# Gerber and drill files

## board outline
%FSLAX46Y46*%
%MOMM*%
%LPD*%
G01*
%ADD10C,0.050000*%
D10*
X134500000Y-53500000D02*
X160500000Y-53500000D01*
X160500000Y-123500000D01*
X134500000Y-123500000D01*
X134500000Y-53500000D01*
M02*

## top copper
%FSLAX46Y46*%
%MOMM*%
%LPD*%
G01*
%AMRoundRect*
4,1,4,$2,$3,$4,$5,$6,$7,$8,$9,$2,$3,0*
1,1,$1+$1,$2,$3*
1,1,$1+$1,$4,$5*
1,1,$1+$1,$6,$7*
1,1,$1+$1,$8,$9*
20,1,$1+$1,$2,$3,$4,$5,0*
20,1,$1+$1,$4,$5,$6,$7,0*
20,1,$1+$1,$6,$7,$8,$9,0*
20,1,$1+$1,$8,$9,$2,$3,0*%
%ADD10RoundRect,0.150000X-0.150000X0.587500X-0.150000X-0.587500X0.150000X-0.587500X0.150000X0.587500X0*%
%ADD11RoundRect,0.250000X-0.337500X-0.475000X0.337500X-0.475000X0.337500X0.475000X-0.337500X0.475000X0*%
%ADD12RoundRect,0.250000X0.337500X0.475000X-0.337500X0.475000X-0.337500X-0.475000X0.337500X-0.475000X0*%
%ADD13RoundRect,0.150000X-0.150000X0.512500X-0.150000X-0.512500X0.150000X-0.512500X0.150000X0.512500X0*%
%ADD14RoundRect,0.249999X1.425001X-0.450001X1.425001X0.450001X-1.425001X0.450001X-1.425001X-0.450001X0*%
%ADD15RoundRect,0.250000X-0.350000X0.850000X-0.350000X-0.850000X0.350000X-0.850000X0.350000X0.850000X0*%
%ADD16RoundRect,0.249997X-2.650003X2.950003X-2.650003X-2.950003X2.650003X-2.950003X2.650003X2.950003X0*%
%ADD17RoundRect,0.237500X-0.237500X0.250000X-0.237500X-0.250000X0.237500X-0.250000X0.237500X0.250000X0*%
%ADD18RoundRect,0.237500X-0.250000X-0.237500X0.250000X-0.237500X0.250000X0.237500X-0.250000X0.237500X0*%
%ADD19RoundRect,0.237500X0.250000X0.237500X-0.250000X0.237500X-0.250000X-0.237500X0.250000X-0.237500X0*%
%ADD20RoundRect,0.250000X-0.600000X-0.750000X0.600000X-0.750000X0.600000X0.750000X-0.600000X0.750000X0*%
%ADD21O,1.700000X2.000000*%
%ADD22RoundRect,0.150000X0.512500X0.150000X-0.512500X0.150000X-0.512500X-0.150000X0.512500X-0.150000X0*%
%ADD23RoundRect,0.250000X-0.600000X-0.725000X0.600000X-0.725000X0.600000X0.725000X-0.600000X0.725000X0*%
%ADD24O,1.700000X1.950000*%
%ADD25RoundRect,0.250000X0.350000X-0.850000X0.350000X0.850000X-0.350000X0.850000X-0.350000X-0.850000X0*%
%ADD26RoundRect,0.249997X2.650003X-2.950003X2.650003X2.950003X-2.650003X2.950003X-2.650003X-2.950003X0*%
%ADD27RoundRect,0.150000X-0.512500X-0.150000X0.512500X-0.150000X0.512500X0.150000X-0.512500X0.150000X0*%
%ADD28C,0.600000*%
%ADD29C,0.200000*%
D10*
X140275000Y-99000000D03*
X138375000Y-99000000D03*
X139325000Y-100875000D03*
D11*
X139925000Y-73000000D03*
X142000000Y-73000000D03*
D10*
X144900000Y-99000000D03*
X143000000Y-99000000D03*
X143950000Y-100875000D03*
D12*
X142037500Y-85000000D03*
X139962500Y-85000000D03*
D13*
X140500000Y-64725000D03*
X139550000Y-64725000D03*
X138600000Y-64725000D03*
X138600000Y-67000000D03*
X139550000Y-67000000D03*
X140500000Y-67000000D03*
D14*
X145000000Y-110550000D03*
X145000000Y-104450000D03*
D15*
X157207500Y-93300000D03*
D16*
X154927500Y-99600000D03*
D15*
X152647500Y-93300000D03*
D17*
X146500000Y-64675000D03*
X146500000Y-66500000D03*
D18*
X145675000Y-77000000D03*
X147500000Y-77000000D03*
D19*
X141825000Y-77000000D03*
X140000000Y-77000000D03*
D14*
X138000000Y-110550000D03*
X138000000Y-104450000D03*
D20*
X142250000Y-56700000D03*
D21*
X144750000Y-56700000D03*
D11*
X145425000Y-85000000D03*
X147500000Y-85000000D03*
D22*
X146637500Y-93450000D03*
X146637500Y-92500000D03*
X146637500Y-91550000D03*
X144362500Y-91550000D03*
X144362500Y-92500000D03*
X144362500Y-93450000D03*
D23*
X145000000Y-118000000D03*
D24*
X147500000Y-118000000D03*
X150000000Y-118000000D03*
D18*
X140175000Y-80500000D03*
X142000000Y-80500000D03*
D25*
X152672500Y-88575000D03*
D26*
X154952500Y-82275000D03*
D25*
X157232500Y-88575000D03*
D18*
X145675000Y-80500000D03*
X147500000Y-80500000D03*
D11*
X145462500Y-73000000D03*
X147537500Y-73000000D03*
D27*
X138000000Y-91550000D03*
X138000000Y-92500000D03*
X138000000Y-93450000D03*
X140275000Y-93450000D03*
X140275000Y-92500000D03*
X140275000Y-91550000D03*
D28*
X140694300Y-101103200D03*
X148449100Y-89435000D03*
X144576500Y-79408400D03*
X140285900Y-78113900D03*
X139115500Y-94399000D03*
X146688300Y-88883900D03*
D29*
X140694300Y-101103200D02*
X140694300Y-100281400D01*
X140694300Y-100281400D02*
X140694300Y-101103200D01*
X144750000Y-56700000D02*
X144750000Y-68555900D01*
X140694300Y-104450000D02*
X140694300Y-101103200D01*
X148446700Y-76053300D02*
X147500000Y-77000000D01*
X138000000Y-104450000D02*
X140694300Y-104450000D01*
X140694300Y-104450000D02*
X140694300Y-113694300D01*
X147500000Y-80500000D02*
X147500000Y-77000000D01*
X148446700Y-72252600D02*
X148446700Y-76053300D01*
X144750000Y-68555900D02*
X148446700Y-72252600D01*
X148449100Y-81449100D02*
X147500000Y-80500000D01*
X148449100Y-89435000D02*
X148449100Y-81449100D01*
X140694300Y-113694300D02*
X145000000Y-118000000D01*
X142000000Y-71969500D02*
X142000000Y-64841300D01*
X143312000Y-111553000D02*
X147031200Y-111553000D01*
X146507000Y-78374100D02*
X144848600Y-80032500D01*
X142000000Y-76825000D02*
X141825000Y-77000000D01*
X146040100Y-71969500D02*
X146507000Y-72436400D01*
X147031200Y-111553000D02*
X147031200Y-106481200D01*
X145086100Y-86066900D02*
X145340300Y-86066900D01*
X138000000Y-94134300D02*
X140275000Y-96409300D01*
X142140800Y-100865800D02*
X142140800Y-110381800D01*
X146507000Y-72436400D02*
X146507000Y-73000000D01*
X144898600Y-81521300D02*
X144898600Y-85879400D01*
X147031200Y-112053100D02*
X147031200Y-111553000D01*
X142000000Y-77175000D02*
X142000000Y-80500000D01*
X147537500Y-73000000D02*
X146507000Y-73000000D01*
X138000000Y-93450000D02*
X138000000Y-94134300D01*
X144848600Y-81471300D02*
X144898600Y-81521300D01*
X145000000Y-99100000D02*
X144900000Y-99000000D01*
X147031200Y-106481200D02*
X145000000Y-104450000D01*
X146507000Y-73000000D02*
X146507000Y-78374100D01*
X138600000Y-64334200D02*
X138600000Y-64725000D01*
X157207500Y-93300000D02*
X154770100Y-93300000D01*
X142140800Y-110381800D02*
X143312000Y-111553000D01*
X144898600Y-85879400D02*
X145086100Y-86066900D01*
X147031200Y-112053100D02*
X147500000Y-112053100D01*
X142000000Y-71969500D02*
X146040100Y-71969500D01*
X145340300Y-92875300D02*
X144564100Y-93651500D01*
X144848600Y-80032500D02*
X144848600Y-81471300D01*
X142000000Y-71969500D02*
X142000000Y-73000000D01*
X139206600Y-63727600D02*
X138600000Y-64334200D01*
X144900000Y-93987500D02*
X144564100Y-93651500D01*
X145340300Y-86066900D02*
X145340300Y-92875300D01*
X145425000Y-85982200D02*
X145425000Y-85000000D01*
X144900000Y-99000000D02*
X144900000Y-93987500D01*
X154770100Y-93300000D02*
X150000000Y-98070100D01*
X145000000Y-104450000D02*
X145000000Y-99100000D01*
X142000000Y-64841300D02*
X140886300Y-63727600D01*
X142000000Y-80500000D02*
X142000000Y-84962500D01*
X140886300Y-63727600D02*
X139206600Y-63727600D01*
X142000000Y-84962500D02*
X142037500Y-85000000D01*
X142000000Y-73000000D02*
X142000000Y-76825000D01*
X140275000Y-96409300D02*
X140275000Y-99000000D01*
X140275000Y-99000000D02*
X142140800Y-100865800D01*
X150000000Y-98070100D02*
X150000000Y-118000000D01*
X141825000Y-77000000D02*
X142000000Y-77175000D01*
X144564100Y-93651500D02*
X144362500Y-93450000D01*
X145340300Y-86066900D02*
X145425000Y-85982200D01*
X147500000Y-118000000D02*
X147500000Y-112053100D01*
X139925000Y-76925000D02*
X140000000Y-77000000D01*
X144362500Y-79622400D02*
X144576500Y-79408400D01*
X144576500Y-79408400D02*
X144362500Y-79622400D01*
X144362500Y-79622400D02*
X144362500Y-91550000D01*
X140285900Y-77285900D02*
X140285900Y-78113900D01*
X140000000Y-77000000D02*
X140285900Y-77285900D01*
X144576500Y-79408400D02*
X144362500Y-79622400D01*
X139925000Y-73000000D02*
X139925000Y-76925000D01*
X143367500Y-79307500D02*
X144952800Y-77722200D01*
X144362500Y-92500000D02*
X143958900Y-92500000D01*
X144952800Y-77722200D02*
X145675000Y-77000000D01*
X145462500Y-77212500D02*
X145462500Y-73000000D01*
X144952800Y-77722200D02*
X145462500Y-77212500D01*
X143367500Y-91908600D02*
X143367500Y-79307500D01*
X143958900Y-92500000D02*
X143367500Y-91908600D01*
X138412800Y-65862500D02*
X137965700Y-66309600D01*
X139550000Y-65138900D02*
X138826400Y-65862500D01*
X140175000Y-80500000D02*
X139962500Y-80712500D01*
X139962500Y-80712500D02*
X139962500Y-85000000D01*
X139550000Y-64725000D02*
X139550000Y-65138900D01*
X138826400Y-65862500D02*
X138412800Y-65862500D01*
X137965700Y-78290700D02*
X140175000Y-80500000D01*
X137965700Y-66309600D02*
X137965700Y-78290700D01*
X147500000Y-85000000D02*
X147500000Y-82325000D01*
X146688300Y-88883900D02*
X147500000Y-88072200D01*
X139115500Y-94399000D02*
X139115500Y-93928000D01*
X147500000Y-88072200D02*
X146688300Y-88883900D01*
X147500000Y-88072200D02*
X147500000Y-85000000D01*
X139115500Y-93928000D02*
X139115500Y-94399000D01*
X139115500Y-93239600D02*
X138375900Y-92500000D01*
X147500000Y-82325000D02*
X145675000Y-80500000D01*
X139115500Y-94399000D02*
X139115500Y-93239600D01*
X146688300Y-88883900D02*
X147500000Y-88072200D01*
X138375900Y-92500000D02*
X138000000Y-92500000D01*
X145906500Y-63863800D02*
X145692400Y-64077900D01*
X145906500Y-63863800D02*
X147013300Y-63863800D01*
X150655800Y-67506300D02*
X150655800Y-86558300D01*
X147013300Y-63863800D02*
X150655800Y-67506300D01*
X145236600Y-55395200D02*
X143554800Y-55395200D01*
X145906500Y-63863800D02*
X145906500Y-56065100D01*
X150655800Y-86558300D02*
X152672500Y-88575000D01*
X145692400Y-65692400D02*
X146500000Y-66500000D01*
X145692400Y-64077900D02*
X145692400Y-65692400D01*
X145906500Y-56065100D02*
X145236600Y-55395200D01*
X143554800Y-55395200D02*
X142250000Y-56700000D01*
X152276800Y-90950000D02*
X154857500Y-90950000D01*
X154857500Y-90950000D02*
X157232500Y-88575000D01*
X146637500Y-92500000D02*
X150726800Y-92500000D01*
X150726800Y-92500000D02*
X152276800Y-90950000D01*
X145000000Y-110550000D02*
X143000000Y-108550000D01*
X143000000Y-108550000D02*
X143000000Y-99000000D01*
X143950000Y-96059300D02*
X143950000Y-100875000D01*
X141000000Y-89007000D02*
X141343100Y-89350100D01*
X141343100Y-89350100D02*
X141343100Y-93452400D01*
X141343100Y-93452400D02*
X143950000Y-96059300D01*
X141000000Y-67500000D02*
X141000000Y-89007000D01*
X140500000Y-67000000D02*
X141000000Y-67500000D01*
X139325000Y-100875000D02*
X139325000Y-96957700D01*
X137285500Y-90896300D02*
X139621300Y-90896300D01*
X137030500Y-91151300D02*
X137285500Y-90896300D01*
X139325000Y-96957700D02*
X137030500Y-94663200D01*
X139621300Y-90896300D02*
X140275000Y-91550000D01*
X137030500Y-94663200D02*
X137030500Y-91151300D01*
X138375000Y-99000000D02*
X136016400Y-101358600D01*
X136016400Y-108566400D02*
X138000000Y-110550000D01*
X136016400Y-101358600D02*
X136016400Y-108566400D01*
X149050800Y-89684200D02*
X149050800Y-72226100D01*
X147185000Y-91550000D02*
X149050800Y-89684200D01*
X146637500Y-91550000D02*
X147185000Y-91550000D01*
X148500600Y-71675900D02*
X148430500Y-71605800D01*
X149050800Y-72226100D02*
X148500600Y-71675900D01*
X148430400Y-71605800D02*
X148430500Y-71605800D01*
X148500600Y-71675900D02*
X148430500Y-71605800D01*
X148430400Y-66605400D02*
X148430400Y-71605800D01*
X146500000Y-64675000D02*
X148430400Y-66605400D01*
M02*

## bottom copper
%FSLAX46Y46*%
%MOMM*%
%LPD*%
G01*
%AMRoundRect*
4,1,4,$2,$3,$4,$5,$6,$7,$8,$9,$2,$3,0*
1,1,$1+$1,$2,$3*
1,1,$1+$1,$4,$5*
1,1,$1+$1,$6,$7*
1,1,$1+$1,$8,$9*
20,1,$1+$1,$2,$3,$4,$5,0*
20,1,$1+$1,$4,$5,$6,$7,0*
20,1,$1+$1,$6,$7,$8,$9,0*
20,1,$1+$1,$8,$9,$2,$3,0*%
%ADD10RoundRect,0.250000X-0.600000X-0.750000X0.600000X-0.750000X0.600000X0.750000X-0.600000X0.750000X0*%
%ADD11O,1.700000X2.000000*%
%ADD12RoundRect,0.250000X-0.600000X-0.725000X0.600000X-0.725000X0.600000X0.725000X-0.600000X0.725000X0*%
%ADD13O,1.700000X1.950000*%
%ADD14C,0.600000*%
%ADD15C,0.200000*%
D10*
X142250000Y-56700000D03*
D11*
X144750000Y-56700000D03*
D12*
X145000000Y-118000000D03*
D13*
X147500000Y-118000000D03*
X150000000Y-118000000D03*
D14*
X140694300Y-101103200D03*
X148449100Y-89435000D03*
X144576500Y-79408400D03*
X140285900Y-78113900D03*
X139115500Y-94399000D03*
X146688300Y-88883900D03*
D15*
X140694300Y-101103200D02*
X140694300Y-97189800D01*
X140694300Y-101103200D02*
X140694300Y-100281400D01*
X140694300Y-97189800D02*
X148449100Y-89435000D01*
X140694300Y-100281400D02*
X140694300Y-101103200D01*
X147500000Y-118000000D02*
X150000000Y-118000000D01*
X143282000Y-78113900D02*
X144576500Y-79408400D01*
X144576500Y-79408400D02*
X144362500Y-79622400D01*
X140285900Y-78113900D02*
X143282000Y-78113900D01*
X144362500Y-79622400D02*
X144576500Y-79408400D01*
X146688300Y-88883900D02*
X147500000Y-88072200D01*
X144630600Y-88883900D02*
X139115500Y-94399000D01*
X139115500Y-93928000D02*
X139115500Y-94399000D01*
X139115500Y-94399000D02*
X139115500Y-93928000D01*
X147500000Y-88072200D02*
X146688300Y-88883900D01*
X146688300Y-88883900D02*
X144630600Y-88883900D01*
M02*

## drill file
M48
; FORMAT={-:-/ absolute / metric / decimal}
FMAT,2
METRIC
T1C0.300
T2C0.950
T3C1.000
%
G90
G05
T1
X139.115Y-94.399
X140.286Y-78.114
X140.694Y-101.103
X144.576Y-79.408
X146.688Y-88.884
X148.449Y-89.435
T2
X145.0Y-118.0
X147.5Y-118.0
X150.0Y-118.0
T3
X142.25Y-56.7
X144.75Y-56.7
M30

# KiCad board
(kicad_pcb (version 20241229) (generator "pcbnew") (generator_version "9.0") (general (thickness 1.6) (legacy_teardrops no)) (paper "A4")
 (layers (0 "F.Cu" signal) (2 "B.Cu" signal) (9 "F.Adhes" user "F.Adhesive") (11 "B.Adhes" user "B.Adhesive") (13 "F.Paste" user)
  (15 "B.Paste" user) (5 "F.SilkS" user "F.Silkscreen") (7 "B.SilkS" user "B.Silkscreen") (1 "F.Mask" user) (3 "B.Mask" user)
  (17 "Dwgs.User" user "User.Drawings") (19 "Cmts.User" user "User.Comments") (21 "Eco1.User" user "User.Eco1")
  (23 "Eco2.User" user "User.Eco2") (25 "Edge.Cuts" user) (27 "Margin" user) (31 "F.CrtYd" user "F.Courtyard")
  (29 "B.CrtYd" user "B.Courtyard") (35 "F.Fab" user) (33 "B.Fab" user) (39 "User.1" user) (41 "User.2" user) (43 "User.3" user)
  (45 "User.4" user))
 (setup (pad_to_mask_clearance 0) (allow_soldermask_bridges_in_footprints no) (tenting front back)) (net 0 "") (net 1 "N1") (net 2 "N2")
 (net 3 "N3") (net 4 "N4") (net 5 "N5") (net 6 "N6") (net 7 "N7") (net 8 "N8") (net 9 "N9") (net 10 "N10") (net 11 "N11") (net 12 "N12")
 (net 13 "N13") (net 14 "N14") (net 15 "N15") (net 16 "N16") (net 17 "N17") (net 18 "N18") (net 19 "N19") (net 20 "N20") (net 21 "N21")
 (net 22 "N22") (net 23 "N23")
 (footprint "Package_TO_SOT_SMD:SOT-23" (layer "F.Cu") (at 139.325 99.9375 -90)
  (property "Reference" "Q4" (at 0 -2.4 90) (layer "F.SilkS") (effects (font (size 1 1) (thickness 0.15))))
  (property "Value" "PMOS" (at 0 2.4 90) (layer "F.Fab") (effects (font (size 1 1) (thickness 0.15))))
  (pad "1" smd roundrect (at -0.9375 -0.95 270) (size 1.475 0.6) (layers "F.Cu" "F.Mask" "F.Paste") (roundrect_rratio 0.25) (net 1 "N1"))
  (pad "2" smd roundrect (at -0.9375 0.95 270) (size 1.475 0.6) (layers "F.Cu" "F.Mask" "F.Paste") (roundrect_rratio 0.25) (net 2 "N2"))
  (pad "3" smd roundrect (at 0.9375 0 270) (size 1.475 0.6) (layers "F.Cu" "F.Mask" "F.Paste") (roundrect_rratio 0.25) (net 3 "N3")))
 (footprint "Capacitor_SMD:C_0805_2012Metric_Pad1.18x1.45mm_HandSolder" (layer "F.Cu") (at 140.9625 73)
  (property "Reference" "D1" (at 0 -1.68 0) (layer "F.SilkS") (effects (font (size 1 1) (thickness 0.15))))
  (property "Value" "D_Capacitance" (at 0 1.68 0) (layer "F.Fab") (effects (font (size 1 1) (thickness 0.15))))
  (pad "1" smd roundrect (at -1.0375 0) (size 1.175 1.45) (layers "F.Cu" "F.Mask" "F.Paste") (roundrect_rratio 0.212766) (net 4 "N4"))
  (pad "2" smd roundrect (at 1.0375 0) (size 1.175 1.45) (layers "F.Cu" "F.Mask" "F.Paste") (roundrect_rratio 0.212766) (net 1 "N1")))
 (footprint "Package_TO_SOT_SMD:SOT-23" (layer "F.Cu") (at 143.95 99.9375 -90)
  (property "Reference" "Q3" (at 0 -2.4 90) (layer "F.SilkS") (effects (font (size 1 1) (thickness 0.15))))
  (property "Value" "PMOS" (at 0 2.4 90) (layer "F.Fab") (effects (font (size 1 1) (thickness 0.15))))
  (pad "1" smd roundrect (at -0.9375 -0.95 270) (size 1.475 0.6) (layers "F.Cu" "F.Mask" "F.Paste") (roundrect_rratio 0.25) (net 1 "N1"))
  (pad "2" smd roundrect (at -0.9375 0.95 270) (size 1.475 0.6) (layers "F.Cu" "F.Mask" "F.Paste") (roundrect_rratio 0.25) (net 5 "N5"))
  (pad "3" smd roundrect (at 0.9375 0 270) (size 1.475 0.6) (layers "F.Cu" "F.Mask" "F.Paste") (roundrect_rratio 0.25) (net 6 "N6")))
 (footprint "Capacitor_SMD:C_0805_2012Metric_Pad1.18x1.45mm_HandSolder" (layer "F.Cu") (at 141 85 180)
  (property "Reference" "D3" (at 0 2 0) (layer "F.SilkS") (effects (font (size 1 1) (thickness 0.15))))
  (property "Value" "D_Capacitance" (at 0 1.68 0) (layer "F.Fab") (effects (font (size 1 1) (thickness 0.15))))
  (pad "1" smd roundrect (at -1.0375 0 180) (size 1.175 1.45) (layers "F.Cu" "F.Mask" "F.Paste") (roundrect_rratio 0.212766) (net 1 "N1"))
  (pad "2" smd roundrect (at 1.0375 0 180) (size 1.175 1.45) (layers "F.Cu" "F.Mask" "F.Paste") (roundrect_rratio 0.212766) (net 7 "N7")))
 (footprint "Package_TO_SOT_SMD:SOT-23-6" (layer "F.Cu") (at 139.55 65.8625 -90)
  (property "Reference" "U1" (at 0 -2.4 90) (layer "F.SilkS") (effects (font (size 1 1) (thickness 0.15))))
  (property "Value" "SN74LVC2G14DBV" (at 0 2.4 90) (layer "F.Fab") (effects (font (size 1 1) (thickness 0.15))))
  (pad "1" smd roundrect (at -1.1375 -0.95 270) (size 1.325 0.6) (layers "F.Cu" "F.Mask" "F.Paste") (roundrect_rratio 0.25) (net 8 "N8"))
  (pad "2" smd roundrect (at -1.1375 0 270) (size 1.325 0.6) (layers "F.Cu" "F.Mask" "F.Paste") (roundrect_rratio 0.25) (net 7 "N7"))
  (pad "3" smd roundrect (at -1.1375 0.95 270) (size 1.325 0.6) (layers "F.Cu" "F.Mask" "F.Paste") (roundrect_rratio 0.25) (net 1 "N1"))
  (pad "4" smd roundrect (at 1.1375 0.95 270) (size 1.325 0.6) (layers "F.Cu" "F.Mask" "F.Paste") (roundrect_rratio 0.25) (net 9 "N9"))
  (pad "5" smd roundrect (at 1.1375 0 270) (size 1.325 0.6) (layers "F.Cu" "F.Mask" "F.Paste") (roundrect_rratio 0.25) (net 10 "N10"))
  (pad "6" smd roundrect (at 1.1375 -0.95 270) (size 1.325 0.6) (layers "F.Cu" "F.Mask" "F.Paste") (roundrect_rratio 0.25) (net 6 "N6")))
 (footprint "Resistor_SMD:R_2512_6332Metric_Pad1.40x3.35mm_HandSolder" (layer "F.Cu") (at 145 107.5 90)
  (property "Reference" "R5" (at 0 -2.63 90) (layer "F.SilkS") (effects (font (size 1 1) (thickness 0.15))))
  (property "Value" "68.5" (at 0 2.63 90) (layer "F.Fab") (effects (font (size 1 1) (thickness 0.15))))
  (pad "1" smd roundrect (at -3.05 0 90) (size 1.4 3.35) (layers "F.Cu" "F.Mask" "F.Paste") (roundrect_rratio 0.178571) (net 5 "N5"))
  (pad "2" smd roundrect (at 3.05 0 90) (size 1.4 3.35) (layers "F.Cu" "F.Mask" "F.Paste") (roundrect_rratio 0.178571) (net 1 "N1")))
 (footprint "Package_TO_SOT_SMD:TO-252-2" (layer "F.Cu") (at 154.9275 98.34 -90)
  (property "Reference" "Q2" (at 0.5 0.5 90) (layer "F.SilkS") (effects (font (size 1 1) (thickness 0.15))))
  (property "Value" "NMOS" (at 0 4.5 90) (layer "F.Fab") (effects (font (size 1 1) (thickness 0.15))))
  (pad "" smd roundrect (at -0.415 -1.525 270) (size 3.05 2.75) (layers "F.Paste") (roundrect_rratio 0.090909))
  (pad "" smd roundrect (at -0.415 1.525 270) (size 3.05 2.75) (layers "F.Paste") (roundrect_rratio 0.090909))
  (pad "" smd roundrect (at 2.935 -1.525 270) (size 3.05 2.75) (layers "F.Paste") (roundrect_rratio 0.090909))
  (pad "" smd roundrect (at 2.935 1.525 270) (size 3.05 2.75) (layers "F.Paste") (roundrect_rratio 0.090909))
  (pad "1" smd roundrect (at -5.04 -2.28 270) (size 2.2 1.2) (layers "F.Cu" "F.Mask" "F.Paste") (roundrect_rratio 0.208333) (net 1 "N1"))
  (pad "2" smd roundrect (at 1.26 0 270) (size 6.4 5.8) (layers "F.Cu" "F.Mask") (roundrect_rratio 0.043103) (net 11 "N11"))
  (pad "3" smd roundrect (at -5.04 2.28 270) (size 2.2 1.2) (layers "F.Cu" "F.Mask" "F.Paste") (roundrect_rratio 0.208333) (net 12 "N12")))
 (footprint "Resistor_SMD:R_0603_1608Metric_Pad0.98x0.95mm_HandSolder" (layer "F.Cu") (at 146.5 65.5875 -90)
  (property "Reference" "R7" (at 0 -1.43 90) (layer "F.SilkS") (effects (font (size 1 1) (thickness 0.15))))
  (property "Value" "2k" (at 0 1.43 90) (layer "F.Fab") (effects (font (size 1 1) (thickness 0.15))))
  (pad "1" smd roundrect (at -0.9125 0 270) (size 0.975 0.95) (layers "F.Cu" "F.Mask" "F.Paste") (roundrect_rratio 0.25) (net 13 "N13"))
  (pad "2" smd roundrect (at 0.9125 0 270) (size 0.975 0.95) (layers "F.Cu" "F.Mask" "F.Paste") (roundrect_rratio 0.25) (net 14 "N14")))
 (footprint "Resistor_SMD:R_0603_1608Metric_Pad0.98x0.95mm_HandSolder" (layer "F.Cu") (at 146.5875 77)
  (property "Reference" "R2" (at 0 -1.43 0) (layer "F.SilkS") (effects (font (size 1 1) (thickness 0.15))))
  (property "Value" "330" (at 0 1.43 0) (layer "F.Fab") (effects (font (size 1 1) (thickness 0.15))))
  (pad "1" smd roundrect (at -0.9125 0) (size 0.975 0.95) (layers "F.Cu" "F.Mask" "F.Paste") (roundrect_rratio 0.25) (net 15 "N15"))
  (pad "2" smd roundrect (at 0.9125 0) (size 0.975 0.95) (layers "F.Cu" "F.Mask" "F.Paste") (roundrect_rratio 0.25) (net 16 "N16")))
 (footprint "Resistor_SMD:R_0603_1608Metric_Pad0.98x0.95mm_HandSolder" (layer "F.Cu") (at 140.9125 77 180)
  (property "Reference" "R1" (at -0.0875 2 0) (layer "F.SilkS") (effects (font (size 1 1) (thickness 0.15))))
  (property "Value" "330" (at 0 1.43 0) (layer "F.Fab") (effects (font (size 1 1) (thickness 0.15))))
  (pad "1" smd roundrect (at -0.9125 0 180) (size 0.975 0.95) (layers "F.Cu" "F.Mask" "F.Paste") (roundrect_rratio 0.25) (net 1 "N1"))
  (pad "2" smd roundrect (at 0.9125 0 180) (size 0.975 0.95) (layers "F.Cu" "F.Mask" "F.Paste") (roundrect_rratio 0.25) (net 4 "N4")))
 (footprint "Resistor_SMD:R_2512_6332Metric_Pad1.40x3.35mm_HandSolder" (layer "F.Cu") (at 138 107.5 90)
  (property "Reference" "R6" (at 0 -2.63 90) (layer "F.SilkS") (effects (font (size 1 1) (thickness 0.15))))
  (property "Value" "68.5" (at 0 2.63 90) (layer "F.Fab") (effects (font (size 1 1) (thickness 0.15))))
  (pad "1" smd roundrect (at -3.05 0 90) (size 1.4 3.35) (layers "F.Cu" "F.Mask" "F.Paste") (roundrect_rratio 0.178571) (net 2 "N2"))
  (pad "2" smd roundrect (at 3.05 0 90) (size 1.4 3.35) (layers "F.Cu" "F.Mask" "F.Paste") (roundrect_rratio 0.178571) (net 16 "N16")))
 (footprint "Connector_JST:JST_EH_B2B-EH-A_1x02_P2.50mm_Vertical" (layer "F.Cu") (at 142.25 56.7)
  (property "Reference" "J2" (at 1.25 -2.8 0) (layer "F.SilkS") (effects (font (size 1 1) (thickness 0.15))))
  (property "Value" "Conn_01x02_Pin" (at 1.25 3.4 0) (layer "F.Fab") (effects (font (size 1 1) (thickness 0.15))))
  (pad "1" thru_hole roundrect (at 0 0) (size 1.7 2) (drill 1) (layers "*.Cu" "*.Mask") (remove_unused_layers no)
   (roundrect_rratio 0.147059) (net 14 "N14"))
  (pad "2" thru_hole oval (at 2.5 0) (size 1.7 2) (drill 1) (layers "*.Cu" "*.Mask") (remove_unused_layers no) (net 16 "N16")))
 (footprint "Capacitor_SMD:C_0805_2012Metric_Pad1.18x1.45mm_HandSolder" (layer "F.Cu") (at 146.4625 85)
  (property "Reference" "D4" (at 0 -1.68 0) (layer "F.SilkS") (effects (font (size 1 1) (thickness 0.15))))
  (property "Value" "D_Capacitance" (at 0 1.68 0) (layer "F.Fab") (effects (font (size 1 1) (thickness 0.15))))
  (pad "1" smd roundrect (at -1.0375 0) (size 1.175 1.45) (layers "F.Cu" "F.Mask" "F.Paste") (roundrect_rratio 0.212766) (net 1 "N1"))
  (pad "2" smd roundrect (at 1.0375 0) (size 1.175 1.45) (layers "F.Cu" "F.Mask" "F.Paste") (roundrect_rratio 0.212766) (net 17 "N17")))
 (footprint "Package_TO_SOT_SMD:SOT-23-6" (layer "F.Cu") (at 145.5 92.5 180)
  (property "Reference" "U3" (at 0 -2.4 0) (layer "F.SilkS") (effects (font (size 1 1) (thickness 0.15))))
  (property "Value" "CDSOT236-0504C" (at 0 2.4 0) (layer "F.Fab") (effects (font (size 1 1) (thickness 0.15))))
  (pad "1" smd roundrect (at -1.1375 -0.95 180) (size 1.325 0.6) (layers "F.Cu" "F.Mask" "F.Paste") (roundrect_rratio 0.25) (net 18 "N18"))
  (pad "2" smd roundrect (at -1.1375 0 180) (size 1.325 0.6) (layers "F.Cu" "F.Mask" "F.Paste") (roundrect_rratio 0.25) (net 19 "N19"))
  (pad "3" smd roundrect (at -1.1375 0.95 180) (size 1.325 0.6) (layers "F.Cu" "F.Mask" "F.Paste") (roundrect_rratio 0.25) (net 13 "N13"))
  (pad "4" smd roundrect (at 1.1375 0.95 180) (size 1.325 0.6) (layers "F.Cu" "F.Mask" "F.Paste") (roundrect_rratio 0.25) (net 4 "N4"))
  (pad "5" smd roundrect (at 1.1375 0 180) (size 1.325 0.6) (layers "F.Cu" "F.Mask" "F.Paste") (roundrect_rratio 0.25) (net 15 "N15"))
  (pad "6" smd roundrect (at 1.1375 -0.95 180) (size 1.325 0.6) (layers "F.Cu" "F.Mask" "F.Paste") (roundrect_rratio 0.25) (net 1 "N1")))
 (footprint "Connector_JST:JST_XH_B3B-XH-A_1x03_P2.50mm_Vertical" (layer "F.Cu") (at 145 118)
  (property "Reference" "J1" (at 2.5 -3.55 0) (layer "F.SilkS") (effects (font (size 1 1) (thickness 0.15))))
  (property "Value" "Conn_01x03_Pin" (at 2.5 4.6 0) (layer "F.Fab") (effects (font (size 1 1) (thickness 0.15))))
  (pad "1" thru_hole roundrect (at 0 0) (size 1.7 1.95) (drill 0.95) (layers "*.Cu" "*.Mask") (remove_unused_layers no)
   (roundrect_rratio 0.147059) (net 16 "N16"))
  (pad "2" thru_hole oval (at 2.5 0) (size 1.7 1.95) (drill 0.95) (layers "*.Cu" "*.Mask") (remove_unused_layers no) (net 1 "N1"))
  (pad "3" thru_hole oval (at 5 0) (size 1.7 1.95) (drill 0.95) (layers "*.Cu" "*.Mask") (remove_unused_layers no) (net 1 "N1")))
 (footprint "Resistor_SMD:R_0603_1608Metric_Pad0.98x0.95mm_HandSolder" (layer "F.Cu") (at 141.0875 80.5)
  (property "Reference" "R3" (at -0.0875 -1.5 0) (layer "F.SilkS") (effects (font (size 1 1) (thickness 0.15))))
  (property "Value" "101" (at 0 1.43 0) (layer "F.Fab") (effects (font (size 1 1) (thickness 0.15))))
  (pad "1" smd roundrect (at -0.9125 0) (size 0.975 0.95) (layers "F.Cu" "F.Mask" "F.Paste") (roundrect_rratio 0.25) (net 7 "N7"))
  (pad "2" smd roundrect (at 0.9125 0) (size 0.975 0.95) (layers "F.Cu" "F.Mask" "F.Paste") (roundrect_rratio 0.25) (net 1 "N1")))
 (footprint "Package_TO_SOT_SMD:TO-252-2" (layer "F.Cu") (at 154.9525 83.535 90)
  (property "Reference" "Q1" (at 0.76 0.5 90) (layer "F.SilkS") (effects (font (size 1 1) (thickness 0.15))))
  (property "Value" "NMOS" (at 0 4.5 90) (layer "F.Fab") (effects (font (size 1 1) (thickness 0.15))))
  (pad "" smd roundrect (at -0.415 -1.525 90) (size 3.05 2.75) (layers "F.Paste") (roundrect_rratio 0.090909))
  (pad "" smd roundrect (at -0.415 1.525 90) (size 3.05 2.75) (layers "F.Paste") (roundrect_rratio 0.090909))
  (pad "" smd roundrect (at 2.935 -1.525 90) (size 3.05 2.75) (layers "F.Paste") (roundrect_rratio 0.090909))
  (pad "" smd roundrect (at 2.935 1.525 90) (size 3.05 2.75) (layers "F.Paste") (roundrect_rratio 0.090909))
  (pad "1" smd roundrect (at -5.04 -2.28 90) (size 2.2 1.2) (layers "F.Cu" "F.Mask" "F.Paste") (roundrect_rratio 0.208333) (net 14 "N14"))
  (pad "2" smd roundrect (at 1.26 0 90) (size 6.4 5.8) (layers "F.Cu" "F.Mask") (roundrect_rratio 0.043103) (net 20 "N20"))
  (pad "3" smd roundrect (at -5.04 2.28 90) (size 2.2 1.2) (layers "F.Cu" "F.Mask" "F.Paste") (roundrect_rratio 0.208333) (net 19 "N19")))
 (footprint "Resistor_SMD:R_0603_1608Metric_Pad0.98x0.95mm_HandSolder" (layer "F.Cu") (at 146.5875 80.5)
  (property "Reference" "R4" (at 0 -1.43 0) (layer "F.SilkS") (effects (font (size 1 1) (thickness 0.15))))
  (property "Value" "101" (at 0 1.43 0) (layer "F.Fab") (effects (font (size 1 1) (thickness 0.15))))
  (pad "1" smd roundrect (at -0.9125 0) (size 0.975 0.95) (layers "F.Cu" "F.Mask" "F.Paste") (roundrect_rratio 0.25) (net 17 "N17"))
  (pad "2" smd roundrect (at 0.9125 0) (size 0.975 0.95) (layers "F.Cu" "F.Mask" "F.Paste") (roundrect_rratio 0.25) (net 16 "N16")))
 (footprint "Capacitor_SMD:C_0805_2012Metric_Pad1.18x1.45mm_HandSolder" (layer "F.Cu") (at 146.5 73)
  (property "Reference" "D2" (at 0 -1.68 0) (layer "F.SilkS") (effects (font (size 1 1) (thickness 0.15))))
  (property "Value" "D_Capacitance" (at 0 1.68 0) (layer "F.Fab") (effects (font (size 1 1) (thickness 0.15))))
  (pad "1" smd roundrect (at -1.0375 0) (size 1.175 1.45) (layers "F.Cu" "F.Mask" "F.Paste") (roundrect_rratio 0.212766) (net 15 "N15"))
  (pad "2" smd roundrect (at 1.0375 0) (size 1.175 1.45) (layers "F.Cu" "F.Mask" "F.Paste") (roundrect_rratio 0.212766) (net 1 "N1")))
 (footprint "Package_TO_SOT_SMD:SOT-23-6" (layer "F.Cu") (at 139.1375 92.5)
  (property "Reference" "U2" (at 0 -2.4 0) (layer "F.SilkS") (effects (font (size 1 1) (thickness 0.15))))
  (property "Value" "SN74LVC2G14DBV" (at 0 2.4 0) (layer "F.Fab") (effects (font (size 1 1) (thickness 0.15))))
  (pad "1" smd roundrect (at -1.1375 -0.95) (size 1.325 0.6) (layers "F.Cu" "F.Mask" "F.Paste") (roundrect_rratio 0.25) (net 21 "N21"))
  (pad "2" smd roundrect (at -1.1375 0) (size 1.325 0.6) (layers "F.Cu" "F.Mask" "F.Paste") (roundrect_rratio 0.25) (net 17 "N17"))
  (pad "3" smd roundrect (at -1.1375 0.95) (size 1.325 0.6) (layers "F.Cu" "F.Mask" "F.Paste") (roundrect_rratio 0.25) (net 1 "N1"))
  (pad "4" smd roundrect (at 1.1375 0.95) (size 1.325 0.6) (layers "F.Cu" "F.Mask" "F.Paste") (roundrect_rratio 0.25) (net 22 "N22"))
  (pad "5" smd roundrect (at 1.1375 0) (size 1.325 0.6) (layers "F.Cu" "F.Mask" "F.Paste") (roundrect_rratio 0.25) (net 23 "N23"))
  (pad "6" smd roundrect (at 1.1375 -0.95) (size 1.325 0.6) (layers "F.Cu" "F.Mask" "F.Paste") (roundrect_rratio 0.25) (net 3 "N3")))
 (gr_rect (start 134.5 53.5) (end 160.5 123.5) (stroke (width 0.05) (type default)) (fill no) (layer "Edge.Cuts"))
 (segment (start 140.6943 101.1032) (end 140.6943 100.2814) (width 0.2) (layer "F.Cu") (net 16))
 (segment (start 140.6943 100.2814) (end 140.6943 101.1032) (width 0.2) (layer "F.Cu") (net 16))
 (segment (start 144.75 56.7) (end 144.75 68.5559) (width 0.2) (layer "F.Cu") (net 16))
 (segment (start 140.6943 104.45) (end 140.6943 101.1032) (width 0.2) (layer "F.Cu") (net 16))
 (segment (start 148.4467 76.0533) (end 147.5 77) (width 0.2) (layer "F.Cu") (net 16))
 (segment (start 138 104.45) (end 140.6943 104.45) (width 0.2) (layer "F.Cu") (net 16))
 (segment (start 140.6943 104.45) (end 140.6943 113.6943) (width 0.2) (layer "F.Cu") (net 16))
 (segment (start 147.5 80.5) (end 147.5 77) (width 0.2) (layer "F.Cu") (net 16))
 (segment (start 148.4467 72.2526) (end 148.4467 76.0533) (width 0.2) (layer "F.Cu") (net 16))
 (segment (start 144.75 68.5559) (end 148.4467 72.2526) (width 0.2) (layer "F.Cu") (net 16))
 (segment (start 148.4491 81.4491) (end 147.5 80.5) (width 0.2) (layer "F.Cu") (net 16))
 (segment (start 148.4491 89.435) (end 148.4491 81.4491) (width 0.2) (layer "F.Cu") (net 16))
 (segment (start 140.6943 113.6943) (end 145 118) (width 0.2) (layer "F.Cu") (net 16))
 (via (at 140.6943 101.1032) (size 0.6) (drill 0.3) (layers "F.Cu" "B.Cu") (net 16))
 (via (at 148.4491 89.435) (size 0.6) (drill 0.3) (layers "F.Cu" "B.Cu") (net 16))
 (segment (start 140.6943 101.1032) (end 140.6943 97.1898) (width 0.2) (layer "B.Cu") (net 16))
 (segment (start 140.6943 101.1032) (end 140.6943 100.2814) (width 0.2) (layer "B.Cu") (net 16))
 (segment (start 140.6943 97.1898) (end 148.4491 89.435) (width 0.2) (layer "B.Cu") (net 16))
 (segment (start 140.6943 100.2814) (end 140.6943 101.1032) (width 0.2) (layer "B.Cu") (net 16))
 (segment (start 142 71.9695) (end 142 64.8413) (width 0.2) (layer "F.Cu") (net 1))
 (segment (start 143.312 111.553) (end 147.0312 111.553) (width 0.2) (layer "F.Cu") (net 1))
 (segment (start 146.507 78.3741) (end 144.8486 80.0325) (width 0.2) (layer "F.Cu") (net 1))
 (segment (start 142 76.825) (end 141.825 77) (width 0.2) (layer "F.Cu") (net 1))
 (segment (start 146.0401 71.9695) (end 146.507 72.4364) (width 0.2) (layer "F.Cu") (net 1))
 (segment (start 147.0312 111.553) (end 147.0312 106.4812) (width 0.2) (layer "F.Cu") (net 1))
 (segment (start 145.0861 86.0669) (end 145.3403 86.0669) (width 0.2) (layer "F.Cu") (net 1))
 (segment (start 138 94.1343) (end 140.275 96.4093) (width 0.2) (layer "F.Cu") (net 1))
 (segment (start 142.1408 100.8658) (end 142.1408 110.3818) (width 0.2) (layer "F.Cu") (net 1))
 (segment (start 146.507 72.4364) (end 146.507 73) (width 0.2) (layer "F.Cu") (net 1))
 (segment (start 144.8986 81.5213) (end 144.8986 85.8794) (width 0.2) (layer "F.Cu") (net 1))
 (segment (start 147.0312 112.0531) (end 147.0312 111.553) (width 0.2) (layer "F.Cu") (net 1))
 (segment (start 142 77.175) (end 142 80.5) (width 0.2) (layer "F.Cu") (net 1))
 (segment (start 147.5375 73) (end 146.507 73) (width 0.2) (layer "F.Cu") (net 1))
 (segment (start 138 93.45) (end 138 94.1343) (width 0.2) (layer "F.Cu") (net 1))
 (segment (start 144.8486 81.4713) (end 144.8986 81.5213) (width 0.2) (layer "F.Cu") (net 1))
 (segment (start 145 99.1) (end 144.9 99) (width 0.2) (layer "F.Cu") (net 1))
 (segment (start 147.0312 106.4812) (end 145 104.45) (width 0.2) (layer "F.Cu") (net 1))
 (segment (start 146.507 73) (end 146.507 78.3741) (width 0.2) (layer "F.Cu") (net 1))
 (segment (start 138.6 64.3342) (end 138.6 64.725) (width 0.2) (layer "F.Cu") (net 1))
 (segment (start 157.2075 93.3) (end 154.7701 93.3) (width 0.2) (layer "F.Cu") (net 1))
 (segment (start 142.1408 110.3818) (end 143.312 111.553) (width 0.2) (layer "F.Cu") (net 1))
 (segment (start 144.8986 85.8794) (end 145.0861 86.0669) (width 0.2) (layer "F.Cu") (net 1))
 (segment (start 147.0312 112.0531) (end 147.5 112.0531) (width 0.2) (layer "F.Cu") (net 1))
 (segment (start 142 71.9695) (end 146.0401 71.9695) (width 0.2) (layer "F.Cu") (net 1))
 (segment (start 145.3403 92.8753) (end 144.5641 93.6515) (width 0.2) (layer "F.Cu") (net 1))
 (segment (start 144.8486 80.0325) (end 144.8486 81.4713) (width 0.2) (layer "F.Cu") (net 1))
 (segment (start 142 71.9695) (end 142 73) (width 0.2) (layer "F.Cu") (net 1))
 (segment (start 139.2066 63.7276) (end 138.6 64.3342) (width 0.2) (layer "F.Cu") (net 1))
 (segment (start 144.9 93.9875) (end 144.5641 93.6515) (width 0.2) (layer "F.Cu") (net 1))
 (segment (start 145.3403 86.0669) (end 145.3403 92.8753) (width 0.2) (layer "F.Cu") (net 1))
 (segment (start 145.425 85.9822) (end 145.425 85) (width 0.2) (layer "F.Cu") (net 1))
 (segment (start 144.9 99) (end 144.9 93.9875) (width 0.2) (layer "F.Cu") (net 1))
 (segment (start 154.7701 93.3) (end 150 98.0701) (width 0.2) (layer "F.Cu") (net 1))
 (segment (start 145 104.45) (end 145 99.1) (width 0.2) (layer "F.Cu") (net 1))
 (segment (start 142 64.8413) (end 140.8863 63.7276) (width 0.2) (layer "F.Cu") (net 1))
 (segment (start 142 80.5) (end 142 84.9625) (width 0.2) (layer "F.Cu") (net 1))
 (segment (start 140.8863 63.7276) (end 139.2066 63.7276) (width 0.2) (layer "F.Cu") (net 1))
 (segment (start 142 84.9625) (end 142.0375 85) (width 0.2) (layer "F.Cu") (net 1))
 (segment (start 142 73) (end 142 76.825) (width 0.2) (layer "F.Cu") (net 1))
 (segment (start 140.275 96.4093) (end 140.275 99) (width 0.2) (layer "F.Cu") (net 1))
 (segment (start 140.275 99) (end 142.1408 100.8658) (width 0.2) (layer "F.Cu") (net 1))
 (segment (start 150 98.0701) (end 150 118) (width 0.2) (layer "F.Cu") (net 1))
 (segment (start 141.825 77) (end 142 77.175) (width 0.2) (layer "F.Cu") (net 1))
 (segment (start 144.5641 93.6515) (end 144.3625 93.45) (width 0.2) (layer "F.Cu") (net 1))
 (segment (start 145.3403 86.0669) (end 145.425 85.9822) (width 0.2) (layer "F.Cu") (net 1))
 (segment (start 147.5 118) (end 147.5 112.0531) (width 0.2) (layer "F.Cu") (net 1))
 (segment (start 147.5 118) (end 150 118) (width 0.2) (layer "B.Cu") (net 1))
 (segment (start 139.925 76.925) (end 140 77) (width 0.2) (layer "F.Cu") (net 4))
 (segment (start 144.3625 79.6224) (end 144.5765 79.4084) (width 0.2) (layer "F.Cu") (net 4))
 (segment (start 144.5765 79.4084) (end 144.3625 79.6224) (width 0.2) (layer "F.Cu") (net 4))
 (segment (start 144.3625 79.6224) (end 144.3625 91.55) (width 0.2) (layer "F.Cu") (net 4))
 (segment (start 140.2859 77.2859) (end 140.2859 78.1139) (width 0.2) (layer "F.Cu") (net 4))
 (segment (start 140 77) (end 140.2859 77.2859) (width 0.2) (layer "F.Cu") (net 4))
 (segment (start 144.5765 79.4084) (end 144.3625 79.6224) (width 0.2) (layer "F.Cu") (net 4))
 (segment (start 139.925 73) (end 139.925 76.925) (width 0.2) (layer "F.Cu") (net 4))
 (via (at 144.5765 79.4084) (size 0.6) (drill 0.3) (layers "F.Cu" "B.Cu") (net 4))
 (via (at 140.2859 78.1139) (size 0.6) (drill 0.3) (layers "F.Cu" "B.Cu") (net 4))
 (segment (start 143.282 78.1139) (end 144.5765 79.4084) (width 0.2) (layer "B.Cu") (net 4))
 (segment (start 144.5765 79.4084) (end 144.3625 79.6224) (width 0.2) (layer "B.Cu") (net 4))
 (segment (start 140.2859 78.1139) (end 143.282 78.1139) (width 0.2) (layer "B.Cu") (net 4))
 (segment (start 144.3625 79.6224) (end 144.5765 79.4084) (width 0.2) (layer "B.Cu") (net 4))
 (segment (start 143.3675 79.3075) (end 144.9528 77.7222) (width 0.2) (layer "F.Cu") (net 15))
 (segment (start 144.3625 92.5) (end 143.9589 92.5) (width 0.2) (layer "F.Cu") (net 15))
 (segment (start 144.9528 77.7222) (end 145.675 77) (width 0.2) (layer "F.Cu") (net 15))
 (segment (start 145.4625 77.2125) (end 145.4625 73) (width 0.2) (layer "F.Cu") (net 15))
 (segment (start 144.9528 77.7222) (end 145.4625 77.2125) (width 0.2) (layer "F.Cu") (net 15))
 (segment (start 143.3675 91.9086) (end 143.3675 79.3075) (width 0.2) (layer "F.Cu") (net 15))
 (segment (start 143.9589 92.5) (end 143.3675 91.9086) (width 0.2) (layer "F.Cu") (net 15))
 (segment (start 138.4128 65.8625) (end 137.9657 66.3096) (width 0.2) (layer "F.Cu") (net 7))
 (segment (start 139.55 65.1389) (end 138.8264 65.8625) (width 0.2) (layer "F.Cu") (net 7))
 (segment (start 140.175 80.5) (end 139.9625 80.7125) (width 0.2) (layer "F.Cu") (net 7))
 (segment (start 139.9625 80.7125) (end 139.9625 85) (width 0.2) (layer "F.Cu") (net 7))
 (segment (start 139.55 64.725) (end 139.55 65.1389) (width 0.2) (layer "F.Cu") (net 7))
 (segment (start 138.8264 65.8625) (end 138.4128 65.8625) (width 0.2) (layer "F.Cu") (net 7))
 (segment (start 137.9657 78.2907) (end 140.175 80.5) (width 0.2) (layer "F.Cu") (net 7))
 (segment (start 137.9657 66.3096) (end 137.9657 78.2907) (width 0.2) (layer "F.Cu") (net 7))
 (segment (start 147.5 85) (end 147.5 82.325) (width 0.2) (layer "F.Cu") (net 17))
 (segment (start 146.6883 88.8839) (end 147.5 88.0722) (width 0.2) (layer "F.Cu") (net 17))
 (segment (start 139.1155 94.399) (end 139.1155 93.928) (width 0.2) (layer "F.Cu") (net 17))
 (segment (start 147.5 88.0722) (end 146.6883 88.8839) (width 0.2) (layer "F.Cu") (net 17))
 (segment (start 147.5 88.0722) (end 147.5 85) (width 0.2) (layer "F.Cu") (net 17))
 (segment (start 139.1155 93.928) (end 139.1155 94.399) (width 0.2) (layer "F.Cu") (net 17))
 (segment (start 139.1155 93.2396) (end 138.3759 92.5) (width 0.2) (layer "F.Cu") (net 17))
 (segment (start 147.5 82.325) (end 145.675 80.5) (width 0.2) (layer "F.Cu") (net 17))
 (segment (start 139.1155 94.399) (end 139.1155 93.2396) (width 0.2) (layer "F.Cu") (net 17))
 (segment (start 146.6883 88.8839) (end 147.5 88.0722) (width 0.2) (layer "F.Cu") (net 17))
 (segment (start 138.3759 92.5) (end 138 92.5) (width 0.2) (layer "F.Cu") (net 17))
 (via (at 139.1155 94.399) (size 0.6) (drill 0.3) (layers "F.Cu" "B.Cu") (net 17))
 (via (at 146.6883 88.8839) (size 0.6) (drill 0.3) (layers "F.Cu" "B.Cu") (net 17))
 (segment (start 146.6883 88.8839) (end 147.5 88.0722) (width 0.2) (layer "B.Cu") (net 17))
 (segment (start 144.6306 88.8839) (end 139.1155 94.399) (width 0.2) (layer "B.Cu") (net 17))
 (segment (start 139.1155 93.928) (end 139.1155 94.399) (width 0.2) (layer "B.Cu") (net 17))
 (segment (start 139.1155 94.399) (end 139.1155 93.928) (width 0.2) (layer "B.Cu") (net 17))
 (segment (start 147.5 88.0722) (end 146.6883 88.8839) (width 0.2) (layer "B.Cu") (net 17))
 (segment (start 146.6883 88.8839) (end 144.6306 88.8839) (width 0.2) (layer "B.Cu") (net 17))
 (segment (start 145.9065 63.8638) (end 145.6924 64.0779) (width 0.2) (layer "F.Cu") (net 14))
 (segment (start 145.9065 63.8638) (end 147.0133 63.8638) (width 0.2) (layer "F.Cu") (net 14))
 (segment (start 150.6558 67.5063) (end 150.6558 86.5583) (width 0.2) (layer "F.Cu") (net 14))
 (segment (start 147.0133 63.8638) (end 150.6558 67.5063) (width 0.2) (layer "F.Cu") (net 14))
 (segment (start 145.2366 55.3952) (end 143.5548 55.3952) (width 0.2) (layer "F.Cu") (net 14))
 (segment (start 145.9065 63.8638) (end 145.9065 56.0651) (width 0.2) (layer "F.Cu") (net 14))
 (segment (start 150.6558 86.5583) (end 152.6725 88.575) (width 0.2) (layer "F.Cu") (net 14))
 (segment (start 145.6924 65.6924) (end 146.5 66.5) (width 0.2) (layer "F.Cu") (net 14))
 (segment (start 145.6924 64.0779) (end 145.6924 65.6924) (width 0.2) (layer "F.Cu") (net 14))
 (segment (start 145.9065 56.0651) (end 145.2366 55.3952) (width 0.2) (layer "F.Cu") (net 14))
 (segment (start 143.5548 55.3952) (end 142.25 56.7) (width 0.2) (layer "F.Cu") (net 14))
 (segment (start 152.2768 90.95) (end 154.8575 90.95) (width 0.2) (layer "F.Cu") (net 19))
 (segment (start 154.8575 90.95) (end 157.2325 88.575) (width 0.2) (layer "F.Cu") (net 19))
 (segment (start 146.6375 92.5) (end 150.7268 92.5) (width 0.2) (layer "F.Cu") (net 19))
 (segment (start 150.7268 92.5) (end 152.2768 90.95) (width 0.2) (layer "F.Cu") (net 19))
 (segment (start 145 110.55) (end 143 108.55) (width 0.2) (layer "F.Cu") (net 5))
 (segment (start 143 108.55) (end 143 99) (width 0.2) (layer "F.Cu") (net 5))
 (segment (start 143.95 96.0593) (end 143.95 100.875) (width 0.2) (layer "F.Cu") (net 6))
 (segment (start 141 89.007) (end 141.3431 89.3501) (width 0.2) (layer "F.Cu") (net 6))
 (segment (start 141.3431 89.3501) (end 141.3431 93.4524) (width 0.2) (layer "F.Cu") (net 6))
 (segment (start 141.3431 93.4524) (end 143.95 96.0593) (width 0.2) (layer "F.Cu") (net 6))
 (segment (start 141 67.5) (end 141 89.007) (width 0.2) (layer "F.Cu") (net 6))
 (segment (start 140.5 67) (end 141 67.5) (width 0.2) (layer "F.Cu") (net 6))
 (segment (start 139.325 100.875) (end 139.325 96.9577) (width 0.2) (layer "F.Cu") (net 3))
 (segment (start 137.2855 90.8963) (end 139.6213 90.8963) (width 0.2) (layer "F.Cu") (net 3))
 (segment (start 137.0305 91.1513) (end 137.2855 90.8963) (width 0.2) (layer "F.Cu") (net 3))
 (segment (start 139.325 96.9577) (end 137.0305 94.6632) (width 0.2) (layer "F.Cu") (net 3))
 (segment (start 139.6213 90.8963) (end 140.275 91.55) (width 0.2) (layer "F.Cu") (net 3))
 (segment (start 137.0305 94.6632) (end 137.0305 91.1513) (width 0.2) (layer "F.Cu") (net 3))
 (segment (start 138.375 99) (end 136.0164 101.3586) (width 0.2) (layer "F.Cu") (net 2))
 (segment (start 136.0164 108.5664) (end 138 110.55) (width 0.2) (layer "F.Cu") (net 2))
 (segment (start 136.0164 101.3586) (end 136.0164 108.5664) (width 0.2) (layer "F.Cu") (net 2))
 (segment (start 149.0508 89.6842) (end 149.0508 72.2261) (width 0.2) (layer "F.Cu") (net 13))
 (segment (start 147.185 91.55) (end 149.0508 89.6842) (width 0.2) (layer "F.Cu") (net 13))
 (segment (start 146.6375 91.55) (end 147.185 91.55) (width 0.2) (layer "F.Cu") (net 13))
 (segment (start 148.5006 71.6759) (end 148.4305 71.6058) (width 0.2) (layer "F.Cu") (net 13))
 (segment (start 149.0508 72.2261) (end 148.5006 71.6759) (width 0.2) (layer "F.Cu") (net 13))
 (segment (start 148.4304 71.6058) (end 148.4305 71.6058) (width 0.2) (layer "F.Cu") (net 13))
 (segment (start 148.5006 71.6759) (end 148.4305 71.6058) (width 0.2) (layer "F.Cu") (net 13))
 (segment (start 148.4304 66.6054) (end 148.4304 71.6058) (width 0.2) (layer "F.Cu") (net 13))
 (segment (start 146.5 64.675) (end 148.4304 66.6054) (width 0.2) (layer "F.Cu") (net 13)))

